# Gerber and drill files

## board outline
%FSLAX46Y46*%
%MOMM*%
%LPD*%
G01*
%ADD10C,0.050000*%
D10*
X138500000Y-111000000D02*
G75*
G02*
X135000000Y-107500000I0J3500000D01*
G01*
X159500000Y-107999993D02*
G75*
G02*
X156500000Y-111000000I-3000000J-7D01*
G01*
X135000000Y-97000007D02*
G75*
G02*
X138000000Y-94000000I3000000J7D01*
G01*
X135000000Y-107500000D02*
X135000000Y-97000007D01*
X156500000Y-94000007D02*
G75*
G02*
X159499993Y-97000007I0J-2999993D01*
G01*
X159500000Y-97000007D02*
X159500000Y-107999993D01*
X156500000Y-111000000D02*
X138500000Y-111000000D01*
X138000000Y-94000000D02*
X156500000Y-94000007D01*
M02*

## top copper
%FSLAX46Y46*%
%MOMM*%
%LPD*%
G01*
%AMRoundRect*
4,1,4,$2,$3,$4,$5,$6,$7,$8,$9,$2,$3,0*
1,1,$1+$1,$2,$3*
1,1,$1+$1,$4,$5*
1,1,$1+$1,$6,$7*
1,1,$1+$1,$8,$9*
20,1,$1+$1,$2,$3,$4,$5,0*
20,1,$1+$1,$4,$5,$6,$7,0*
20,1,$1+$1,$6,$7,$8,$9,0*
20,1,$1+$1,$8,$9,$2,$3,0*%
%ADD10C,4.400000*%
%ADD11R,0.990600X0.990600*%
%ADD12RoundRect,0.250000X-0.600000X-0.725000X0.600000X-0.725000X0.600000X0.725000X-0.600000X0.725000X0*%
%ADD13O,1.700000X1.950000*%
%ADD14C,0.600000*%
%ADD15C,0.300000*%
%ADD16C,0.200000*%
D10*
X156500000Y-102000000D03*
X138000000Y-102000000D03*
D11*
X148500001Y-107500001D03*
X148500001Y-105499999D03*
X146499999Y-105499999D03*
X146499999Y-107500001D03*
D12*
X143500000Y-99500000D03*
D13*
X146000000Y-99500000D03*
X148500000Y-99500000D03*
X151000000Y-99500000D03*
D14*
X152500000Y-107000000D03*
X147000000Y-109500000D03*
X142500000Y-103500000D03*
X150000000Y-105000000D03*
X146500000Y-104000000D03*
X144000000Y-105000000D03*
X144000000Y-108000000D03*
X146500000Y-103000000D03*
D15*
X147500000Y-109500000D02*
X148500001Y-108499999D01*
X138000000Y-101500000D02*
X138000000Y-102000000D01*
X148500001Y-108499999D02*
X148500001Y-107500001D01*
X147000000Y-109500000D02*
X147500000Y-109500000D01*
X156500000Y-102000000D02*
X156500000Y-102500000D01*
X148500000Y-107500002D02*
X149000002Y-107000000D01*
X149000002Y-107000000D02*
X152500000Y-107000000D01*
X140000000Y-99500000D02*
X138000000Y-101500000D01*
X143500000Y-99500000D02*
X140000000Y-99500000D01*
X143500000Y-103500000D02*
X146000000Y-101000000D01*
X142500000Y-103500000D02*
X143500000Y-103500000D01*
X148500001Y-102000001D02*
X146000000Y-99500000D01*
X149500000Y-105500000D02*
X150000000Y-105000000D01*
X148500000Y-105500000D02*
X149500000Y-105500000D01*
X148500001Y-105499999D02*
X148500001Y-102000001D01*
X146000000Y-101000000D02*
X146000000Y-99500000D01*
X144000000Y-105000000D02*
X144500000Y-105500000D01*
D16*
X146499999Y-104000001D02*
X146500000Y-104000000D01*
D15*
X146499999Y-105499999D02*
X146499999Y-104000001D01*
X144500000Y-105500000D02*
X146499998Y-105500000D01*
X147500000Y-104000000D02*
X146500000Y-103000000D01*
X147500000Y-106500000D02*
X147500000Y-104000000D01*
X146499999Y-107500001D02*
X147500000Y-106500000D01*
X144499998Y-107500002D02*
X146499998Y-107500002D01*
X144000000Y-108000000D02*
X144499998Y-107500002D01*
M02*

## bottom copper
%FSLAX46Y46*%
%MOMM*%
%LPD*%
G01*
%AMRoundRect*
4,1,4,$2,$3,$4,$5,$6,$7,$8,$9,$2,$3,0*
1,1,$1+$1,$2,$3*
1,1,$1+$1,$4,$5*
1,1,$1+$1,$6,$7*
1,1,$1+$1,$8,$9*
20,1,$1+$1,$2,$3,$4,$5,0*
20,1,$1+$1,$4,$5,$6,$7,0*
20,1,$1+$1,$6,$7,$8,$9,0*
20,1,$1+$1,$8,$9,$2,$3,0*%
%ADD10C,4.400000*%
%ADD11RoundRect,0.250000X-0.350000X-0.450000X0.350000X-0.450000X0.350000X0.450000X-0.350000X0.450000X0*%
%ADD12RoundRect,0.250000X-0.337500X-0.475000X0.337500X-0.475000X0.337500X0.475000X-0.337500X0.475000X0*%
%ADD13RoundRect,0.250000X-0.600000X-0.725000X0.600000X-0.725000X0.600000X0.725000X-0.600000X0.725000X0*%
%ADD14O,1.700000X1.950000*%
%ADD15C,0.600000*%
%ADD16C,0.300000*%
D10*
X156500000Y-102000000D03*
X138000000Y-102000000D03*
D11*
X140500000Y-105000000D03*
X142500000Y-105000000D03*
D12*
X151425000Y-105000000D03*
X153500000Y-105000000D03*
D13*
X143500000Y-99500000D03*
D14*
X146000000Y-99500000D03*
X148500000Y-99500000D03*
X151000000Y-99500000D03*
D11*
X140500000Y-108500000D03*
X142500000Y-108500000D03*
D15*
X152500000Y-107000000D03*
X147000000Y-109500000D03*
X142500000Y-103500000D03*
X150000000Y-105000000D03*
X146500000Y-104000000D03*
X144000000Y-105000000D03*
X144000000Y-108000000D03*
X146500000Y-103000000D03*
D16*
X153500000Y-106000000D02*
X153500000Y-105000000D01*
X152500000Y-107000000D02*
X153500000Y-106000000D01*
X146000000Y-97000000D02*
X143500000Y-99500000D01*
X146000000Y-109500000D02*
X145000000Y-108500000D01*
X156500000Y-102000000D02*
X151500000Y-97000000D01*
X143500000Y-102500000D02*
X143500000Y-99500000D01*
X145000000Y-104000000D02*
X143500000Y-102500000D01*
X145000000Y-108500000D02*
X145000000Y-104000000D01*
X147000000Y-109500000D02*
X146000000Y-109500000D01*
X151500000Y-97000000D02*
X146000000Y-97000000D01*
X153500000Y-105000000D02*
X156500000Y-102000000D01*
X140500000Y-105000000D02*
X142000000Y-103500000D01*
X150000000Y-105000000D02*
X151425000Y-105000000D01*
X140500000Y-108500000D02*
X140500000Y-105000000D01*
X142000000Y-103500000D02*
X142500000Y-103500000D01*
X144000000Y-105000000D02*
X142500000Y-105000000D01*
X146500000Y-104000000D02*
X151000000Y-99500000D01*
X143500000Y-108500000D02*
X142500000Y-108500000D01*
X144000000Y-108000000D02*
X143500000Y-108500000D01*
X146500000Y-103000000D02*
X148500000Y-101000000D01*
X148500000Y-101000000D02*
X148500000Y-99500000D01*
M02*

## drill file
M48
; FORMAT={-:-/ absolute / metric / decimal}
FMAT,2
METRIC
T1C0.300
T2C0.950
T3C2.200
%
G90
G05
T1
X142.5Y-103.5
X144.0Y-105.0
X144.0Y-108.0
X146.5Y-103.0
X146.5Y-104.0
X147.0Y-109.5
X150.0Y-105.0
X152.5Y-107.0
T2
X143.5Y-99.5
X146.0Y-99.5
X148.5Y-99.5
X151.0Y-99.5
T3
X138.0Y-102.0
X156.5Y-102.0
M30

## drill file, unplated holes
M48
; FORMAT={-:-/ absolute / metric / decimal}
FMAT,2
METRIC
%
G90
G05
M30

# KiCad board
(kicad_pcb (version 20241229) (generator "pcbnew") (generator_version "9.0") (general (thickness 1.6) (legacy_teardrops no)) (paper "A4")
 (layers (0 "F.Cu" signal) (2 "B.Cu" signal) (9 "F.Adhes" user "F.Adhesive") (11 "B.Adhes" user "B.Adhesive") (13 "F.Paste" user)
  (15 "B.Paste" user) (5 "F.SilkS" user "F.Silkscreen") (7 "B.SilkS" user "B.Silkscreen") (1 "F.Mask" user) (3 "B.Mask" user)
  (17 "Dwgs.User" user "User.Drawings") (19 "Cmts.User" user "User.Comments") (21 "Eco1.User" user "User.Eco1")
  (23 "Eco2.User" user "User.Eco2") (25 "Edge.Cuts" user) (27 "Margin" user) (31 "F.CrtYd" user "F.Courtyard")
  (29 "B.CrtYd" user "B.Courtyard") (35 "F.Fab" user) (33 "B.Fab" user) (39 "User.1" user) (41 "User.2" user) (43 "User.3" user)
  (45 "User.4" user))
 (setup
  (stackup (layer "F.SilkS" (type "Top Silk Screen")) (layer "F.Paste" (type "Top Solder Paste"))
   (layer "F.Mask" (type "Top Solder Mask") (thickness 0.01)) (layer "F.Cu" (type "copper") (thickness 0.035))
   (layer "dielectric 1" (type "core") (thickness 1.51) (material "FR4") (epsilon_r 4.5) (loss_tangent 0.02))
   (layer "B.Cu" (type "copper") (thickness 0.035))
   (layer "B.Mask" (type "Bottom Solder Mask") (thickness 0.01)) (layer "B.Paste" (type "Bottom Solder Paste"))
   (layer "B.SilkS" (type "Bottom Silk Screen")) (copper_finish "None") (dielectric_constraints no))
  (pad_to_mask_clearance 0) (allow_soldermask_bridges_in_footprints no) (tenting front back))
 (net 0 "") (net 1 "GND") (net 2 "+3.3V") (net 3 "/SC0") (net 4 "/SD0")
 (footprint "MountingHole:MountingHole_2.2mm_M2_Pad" (layer "F.Cu") (at 156.5 102)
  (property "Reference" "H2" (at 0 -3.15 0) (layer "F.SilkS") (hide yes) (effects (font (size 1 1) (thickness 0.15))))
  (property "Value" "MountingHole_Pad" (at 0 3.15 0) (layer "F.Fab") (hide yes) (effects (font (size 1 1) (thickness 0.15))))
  (pad "1" thru_hole circle (at 0 0) (size 4.4 4.4) (drill 2.2) (layers "*.Cu" "*.Mask") (remove_unused_layers no) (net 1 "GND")
   (zone_connect 2)))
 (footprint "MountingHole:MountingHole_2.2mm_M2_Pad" (layer "F.Cu") (at 138 102)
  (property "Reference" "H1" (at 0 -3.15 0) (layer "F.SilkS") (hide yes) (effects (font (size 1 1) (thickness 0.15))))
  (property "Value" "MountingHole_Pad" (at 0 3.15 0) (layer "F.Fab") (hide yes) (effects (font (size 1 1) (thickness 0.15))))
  (pad "1" thru_hole circle (at 0 0) (size 4.4 4.4) (drill 2.2) (layers "*.Cu" "*.Mask") (remove_unused_layers no) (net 1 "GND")
   (zone_connect 2)))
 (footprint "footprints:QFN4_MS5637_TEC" (layer "F.Cu") (at 147.5 106.5 180)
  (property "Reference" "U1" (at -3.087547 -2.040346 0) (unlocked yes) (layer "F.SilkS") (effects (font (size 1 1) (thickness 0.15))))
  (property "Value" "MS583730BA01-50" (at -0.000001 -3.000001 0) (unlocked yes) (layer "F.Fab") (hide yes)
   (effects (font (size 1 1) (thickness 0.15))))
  (pad "1" smd rect (at -1.000001 -1.000001 180) (size 0.9906 0.9906) (layers "F.Cu" "F.Mask" "F.Paste") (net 1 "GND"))
  (pad "2" smd rect (at -1.000001 1.000001 180) (size 0.9906 0.9906) (layers "F.Cu" "F.Mask" "F.Paste") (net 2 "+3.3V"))
  (pad "3" smd rect (at 1.000001 1.000001 180) (size 0.9906 0.9906) (layers "F.Cu" "F.Mask" "F.Paste") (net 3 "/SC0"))
  (pad "4" smd rect (at 1.000001 -1.000001 180) (size 0.9906 0.9906) (layers "F.Cu" "F.Mask" "F.Paste") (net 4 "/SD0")))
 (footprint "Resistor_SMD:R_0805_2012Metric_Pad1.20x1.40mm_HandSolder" (layer "B.Cu") (at 141.5 105)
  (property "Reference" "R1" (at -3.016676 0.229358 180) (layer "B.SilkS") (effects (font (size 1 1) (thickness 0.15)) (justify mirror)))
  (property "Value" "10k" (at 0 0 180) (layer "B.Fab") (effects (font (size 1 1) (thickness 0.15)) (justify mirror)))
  (pad "1" smd roundrect (at -1 0) (size 1.2 1.4) (layers "B.Cu" "B.Mask" "B.Paste") (roundrect_rratio 0.208333) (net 2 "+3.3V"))
  (pad "2" smd roundrect (at 1 0) (size 1.2 1.4) (layers "B.Cu" "B.Mask" "B.Paste") (roundrect_rratio 0.208333) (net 3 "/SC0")))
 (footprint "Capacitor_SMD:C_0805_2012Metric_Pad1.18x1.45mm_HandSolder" (layer "B.Cu") (at 152.4625 105)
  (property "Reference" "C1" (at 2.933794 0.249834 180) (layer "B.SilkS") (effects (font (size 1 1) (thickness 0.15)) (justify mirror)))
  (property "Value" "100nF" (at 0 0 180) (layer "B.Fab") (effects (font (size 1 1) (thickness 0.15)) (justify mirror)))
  (pad "1" smd roundrect (at -1.0375 0) (size 1.175 1.45) (layers "B.Cu" "B.Mask" "B.Paste") (roundrect_rratio 0.212766) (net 2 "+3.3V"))
  (pad "2" smd roundrect (at 1.0375 0) (size 1.175 1.45) (layers "B.Cu" "B.Mask" "B.Paste") (roundrect_rratio 0.212766) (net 1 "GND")))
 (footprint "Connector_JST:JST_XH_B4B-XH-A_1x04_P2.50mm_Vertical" (layer "B.Cu") (at 143.5 99.5)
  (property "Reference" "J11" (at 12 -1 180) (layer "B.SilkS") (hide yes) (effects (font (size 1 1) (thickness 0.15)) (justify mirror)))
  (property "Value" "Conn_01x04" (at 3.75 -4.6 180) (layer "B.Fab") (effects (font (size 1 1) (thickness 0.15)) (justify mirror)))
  (pad "1" thru_hole roundrect (at 0 0) (size 1.7 1.95) (drill 0.95) (layers "*.Cu" "*.Mask") (remove_unused_layers no)
   (roundrect_rratio 0.147059) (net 1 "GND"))
  (pad "2" thru_hole oval (at 2.5 0) (size 1.7 1.95) (drill 0.95) (layers "*.Cu" "*.Mask") (remove_unused_layers no) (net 2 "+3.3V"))
  (pad "3" thru_hole oval (at 5 0) (size 1.7 1.95) (drill 0.95) (layers "*.Cu" "*.Mask") (remove_unused_layers no) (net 4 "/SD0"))
  (pad "4" thru_hole oval (at 7.5 0) (size 1.7 1.95) (drill 0.95) (layers "*.Cu" "*.Mask") (remove_unused_layers no) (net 3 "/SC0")))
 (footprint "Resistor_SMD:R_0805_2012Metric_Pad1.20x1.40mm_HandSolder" (layer "B.Cu") (at 141.5 108.5)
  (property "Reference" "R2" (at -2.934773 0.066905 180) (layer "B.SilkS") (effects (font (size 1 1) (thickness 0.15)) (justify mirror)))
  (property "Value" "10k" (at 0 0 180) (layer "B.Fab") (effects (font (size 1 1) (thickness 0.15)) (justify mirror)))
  (pad "1" smd roundrect (at -1 0) (size 1.2 1.4) (layers "B.Cu" "B.Mask" "B.Paste") (roundrect_rratio 0.208333) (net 2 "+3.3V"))
  (pad "2" smd roundrect (at 1 0) (size 1.2 1.4) (layers "B.Cu" "B.Mask" "B.Paste") (roundrect_rratio 0.208333) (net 4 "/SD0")))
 (gr_arc (start 138.5 111) (mid 136.025126 109.974874) (end 135 107.5) (stroke (width 0.05) (type default)) (layer "Edge.Cuts"))
 (gr_arc (start 159.5 107.999993) (mid 158.621323 110.121318) (end 156.5 111) (stroke (width 0.05) (type default)) (layer "Edge.Cuts"))
 (gr_arc (start 135 97.000007) (mid 135.878677 94.878682) (end 138 94) (stroke (width 0.05) (type default)) (layer "Edge.Cuts"))
 (gr_line (start 135 107.5) (end 135 97.000007) (stroke (width 0.05) (type default)) (layer "Edge.Cuts"))
 (gr_arc (start 156.5 94.000007) (mid 158.62132 94.878687) (end 159.5 97.000007) (stroke (width 0.05) (type default)) (layer "Edge.Cuts"))
 (gr_line (start 159.5 97.000007) (end 159.5 107.999993) (stroke (width 0.05) (type default)) (layer "Edge.Cuts"))
 (gr_line (start 156.5 111) (end 138.5 111) (stroke (width 0.05) (type default)) (layer "Edge.Cuts"))
 (gr_line (start 138 94) (end 156.5 94.000007) (stroke (width 0.05) (type solid)) (layer "Edge.Cuts"))
 (segment (start 147.5 109.5) (end 148.500001 108.499999) (width 0.3) (layer "F.Cu") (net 1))
 (segment (start 138 101.5) (end 138 102) (width 0.3) (layer "F.Cu") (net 1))
 (segment (start 148.500001 108.499999) (end 148.500001 107.500001) (width 0.3) (layer "F.Cu") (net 1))
 (segment (start 147 109.5) (end 147.5 109.5) (width 0.3) (layer "F.Cu") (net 1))
 (segment (start 156.5 102) (end 156.5 102.5) (width 0.3) (layer "F.Cu") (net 1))
 (segment (start 148.5 107.500002) (end 149.000002 107) (width 0.3) (layer "F.Cu") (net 1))
 (segment (start 149.000002 107) (end 152.5 107) (width 0.3) (layer "F.Cu") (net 1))
 (segment (start 140 99.5) (end 138 101.5) (width 0.3) (layer "F.Cu") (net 1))
 (segment (start 143.5 99.5) (end 140 99.5) (width 0.3) (layer "F.Cu") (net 1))
 (via (at 152.5 107) (size 0.6) (drill 0.3) (layers "F.Cu" "B.Cu") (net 1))
 (via (at 147 109.5) (size 0.6) (drill 0.3) (layers "F.Cu" "B.Cu") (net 1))
 (segment (start 153.5 106) (end 153.5 105) (width 0.3) (layer "B.Cu") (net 1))
 (segment (start 152.5 107) (end 153.5 106) (width 0.3) (layer "B.Cu") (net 1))
 (segment (start 146 97) (end 143.5 99.5) (width 0.3) (layer "B.Cu") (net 1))
 (segment (start 146 109.5) (end 145 108.5) (width 0.3) (layer "B.Cu") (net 1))
 (segment (start 156.5 102) (end 151.5 97) (width 0.3) (layer "B.Cu") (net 1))
 (segment (start 143.5 102.5) (end 143.5 99.5) (width 0.3) (layer "B.Cu") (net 1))
 (segment (start 145 104) (end 143.5 102.5) (width 0.3) (layer "B.Cu") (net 1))
 (segment (start 145 108.5) (end 145 104) (width 0.3) (layer "B.Cu") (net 1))
 (segment (start 147 109.5) (end 146 109.5) (width 0.3) (layer "B.Cu") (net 1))
 (segment (start 151.5 97) (end 146 97) (width 0.3) (layer "B.Cu") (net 1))
 (segment (start 153.5 105) (end 156.5 102) (width 0.3) (layer "B.Cu") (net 1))
 (segment (start 143.5 103.5) (end 146 101) (width 0.3) (layer "F.Cu") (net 2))
 (segment (start 142.5 103.5) (end 143.5 103.5) (width 0.3) (layer "F.Cu") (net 2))
 (segment (start 148.500001 102.000001) (end 146 99.5) (width 0.3) (layer "F.Cu") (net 2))
 (segment (start 149.5 105.5) (end 150 105) (width 0.3) (layer "F.Cu") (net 2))
 (segment (start 148.5 105.5) (end 149.5 105.5) (width 0.3) (layer "F.Cu") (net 2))
 (segment (start 148.500001 105.499999) (end 148.500001 102.000001) (width 0.3) (layer "F.Cu") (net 2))
 (segment (start 146 101) (end 146 99.5) (width 0.3) (layer "F.Cu") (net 2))
 (via (at 142.5 103.5) (size 0.6) (drill 0.3) (layers "F.Cu" "B.Cu") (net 2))
 (via (at 150 105) (size 0.6) (drill 0.3) (layers "F.Cu" "B.Cu") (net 2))
 (segment (start 140.5 105) (end 142 103.5) (width 0.3) (layer "B.Cu") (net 2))
 (segment (start 150 105) (end 151.425 105) (width 0.3) (layer "B.Cu") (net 2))
 (segment (start 140.5 108.5) (end 140.5 105) (width 0.3) (layer "B.Cu") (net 2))
 (segment (start 142 103.5) (end 142.5 103.5) (width 0.3) (layer "B.Cu") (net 2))
 (segment (start 144 105) (end 144.5 105.5) (width 0.3) (layer "F.Cu") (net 3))
 (segment (start 146.499999 104.000001) (end 146.5 104) (width 0.2) (layer "F.Cu") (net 3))
 (segment (start 146.499999 105.499999) (end 146.499999 104.000001) (width 0.3) (layer "F.Cu") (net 3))
 (segment (start 144.5 105.5) (end 146.499998 105.5) (width 0.3) (layer "F.Cu") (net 3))
 (via (at 146.5 104) (size 0.6) (drill 0.3) (layers "F.Cu" "B.Cu") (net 3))
 (via (at 144 105) (size 0.6) (drill 0.3) (layers "F.Cu" "B.Cu") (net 3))
 (segment (start 144 105) (end 142.5 105) (width 0.3) (layer "B.Cu") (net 3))
 (segment (start 146.5 104) (end 151 99.5) (width 0.3) (layer "B.Cu") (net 3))
 (segment (start 147.5 104) (end 146.5 103) (width 0.3) (layer "F.Cu") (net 4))
 (segment (start 147.5 106.5) (end 147.5 104) (width 0.3) (layer "F.Cu") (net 4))
 (segment (start 146.499999 107.500001) (end 147.5 106.5) (width 0.3) (layer "F.Cu") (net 4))
 (segment (start 144.499998 107.500002) (end 146.499998 107.500002) (width 0.3) (layer "F.Cu") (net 4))
 (segment (start 144 108) (end 144.499998 107.500002) (width 0.3) (layer "F.Cu") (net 4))
 (via (at 144 108) (size 0.6) (drill 0.3) (layers "F.Cu" "B.Cu") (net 4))
 (via (at 146.5 103) (size 0.6) (drill 0.3) (layers "F.Cu" "B.Cu") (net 4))
 (segment (start 143.5 108.5) (end 142.5 108.5) (width 0.3) (layer "B.Cu") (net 4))
 (segment (start 144 108) (end 143.5 108.5) (width 0.3) (layer "B.Cu") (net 4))
 (segment (start 146.5 103) (end 148.5 101) (width 0.3) (layer "B.Cu") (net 4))
 (segment (start 148.5 101) (end 148.5 99.5) (width 0.3) (layer "B.Cu") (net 4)))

